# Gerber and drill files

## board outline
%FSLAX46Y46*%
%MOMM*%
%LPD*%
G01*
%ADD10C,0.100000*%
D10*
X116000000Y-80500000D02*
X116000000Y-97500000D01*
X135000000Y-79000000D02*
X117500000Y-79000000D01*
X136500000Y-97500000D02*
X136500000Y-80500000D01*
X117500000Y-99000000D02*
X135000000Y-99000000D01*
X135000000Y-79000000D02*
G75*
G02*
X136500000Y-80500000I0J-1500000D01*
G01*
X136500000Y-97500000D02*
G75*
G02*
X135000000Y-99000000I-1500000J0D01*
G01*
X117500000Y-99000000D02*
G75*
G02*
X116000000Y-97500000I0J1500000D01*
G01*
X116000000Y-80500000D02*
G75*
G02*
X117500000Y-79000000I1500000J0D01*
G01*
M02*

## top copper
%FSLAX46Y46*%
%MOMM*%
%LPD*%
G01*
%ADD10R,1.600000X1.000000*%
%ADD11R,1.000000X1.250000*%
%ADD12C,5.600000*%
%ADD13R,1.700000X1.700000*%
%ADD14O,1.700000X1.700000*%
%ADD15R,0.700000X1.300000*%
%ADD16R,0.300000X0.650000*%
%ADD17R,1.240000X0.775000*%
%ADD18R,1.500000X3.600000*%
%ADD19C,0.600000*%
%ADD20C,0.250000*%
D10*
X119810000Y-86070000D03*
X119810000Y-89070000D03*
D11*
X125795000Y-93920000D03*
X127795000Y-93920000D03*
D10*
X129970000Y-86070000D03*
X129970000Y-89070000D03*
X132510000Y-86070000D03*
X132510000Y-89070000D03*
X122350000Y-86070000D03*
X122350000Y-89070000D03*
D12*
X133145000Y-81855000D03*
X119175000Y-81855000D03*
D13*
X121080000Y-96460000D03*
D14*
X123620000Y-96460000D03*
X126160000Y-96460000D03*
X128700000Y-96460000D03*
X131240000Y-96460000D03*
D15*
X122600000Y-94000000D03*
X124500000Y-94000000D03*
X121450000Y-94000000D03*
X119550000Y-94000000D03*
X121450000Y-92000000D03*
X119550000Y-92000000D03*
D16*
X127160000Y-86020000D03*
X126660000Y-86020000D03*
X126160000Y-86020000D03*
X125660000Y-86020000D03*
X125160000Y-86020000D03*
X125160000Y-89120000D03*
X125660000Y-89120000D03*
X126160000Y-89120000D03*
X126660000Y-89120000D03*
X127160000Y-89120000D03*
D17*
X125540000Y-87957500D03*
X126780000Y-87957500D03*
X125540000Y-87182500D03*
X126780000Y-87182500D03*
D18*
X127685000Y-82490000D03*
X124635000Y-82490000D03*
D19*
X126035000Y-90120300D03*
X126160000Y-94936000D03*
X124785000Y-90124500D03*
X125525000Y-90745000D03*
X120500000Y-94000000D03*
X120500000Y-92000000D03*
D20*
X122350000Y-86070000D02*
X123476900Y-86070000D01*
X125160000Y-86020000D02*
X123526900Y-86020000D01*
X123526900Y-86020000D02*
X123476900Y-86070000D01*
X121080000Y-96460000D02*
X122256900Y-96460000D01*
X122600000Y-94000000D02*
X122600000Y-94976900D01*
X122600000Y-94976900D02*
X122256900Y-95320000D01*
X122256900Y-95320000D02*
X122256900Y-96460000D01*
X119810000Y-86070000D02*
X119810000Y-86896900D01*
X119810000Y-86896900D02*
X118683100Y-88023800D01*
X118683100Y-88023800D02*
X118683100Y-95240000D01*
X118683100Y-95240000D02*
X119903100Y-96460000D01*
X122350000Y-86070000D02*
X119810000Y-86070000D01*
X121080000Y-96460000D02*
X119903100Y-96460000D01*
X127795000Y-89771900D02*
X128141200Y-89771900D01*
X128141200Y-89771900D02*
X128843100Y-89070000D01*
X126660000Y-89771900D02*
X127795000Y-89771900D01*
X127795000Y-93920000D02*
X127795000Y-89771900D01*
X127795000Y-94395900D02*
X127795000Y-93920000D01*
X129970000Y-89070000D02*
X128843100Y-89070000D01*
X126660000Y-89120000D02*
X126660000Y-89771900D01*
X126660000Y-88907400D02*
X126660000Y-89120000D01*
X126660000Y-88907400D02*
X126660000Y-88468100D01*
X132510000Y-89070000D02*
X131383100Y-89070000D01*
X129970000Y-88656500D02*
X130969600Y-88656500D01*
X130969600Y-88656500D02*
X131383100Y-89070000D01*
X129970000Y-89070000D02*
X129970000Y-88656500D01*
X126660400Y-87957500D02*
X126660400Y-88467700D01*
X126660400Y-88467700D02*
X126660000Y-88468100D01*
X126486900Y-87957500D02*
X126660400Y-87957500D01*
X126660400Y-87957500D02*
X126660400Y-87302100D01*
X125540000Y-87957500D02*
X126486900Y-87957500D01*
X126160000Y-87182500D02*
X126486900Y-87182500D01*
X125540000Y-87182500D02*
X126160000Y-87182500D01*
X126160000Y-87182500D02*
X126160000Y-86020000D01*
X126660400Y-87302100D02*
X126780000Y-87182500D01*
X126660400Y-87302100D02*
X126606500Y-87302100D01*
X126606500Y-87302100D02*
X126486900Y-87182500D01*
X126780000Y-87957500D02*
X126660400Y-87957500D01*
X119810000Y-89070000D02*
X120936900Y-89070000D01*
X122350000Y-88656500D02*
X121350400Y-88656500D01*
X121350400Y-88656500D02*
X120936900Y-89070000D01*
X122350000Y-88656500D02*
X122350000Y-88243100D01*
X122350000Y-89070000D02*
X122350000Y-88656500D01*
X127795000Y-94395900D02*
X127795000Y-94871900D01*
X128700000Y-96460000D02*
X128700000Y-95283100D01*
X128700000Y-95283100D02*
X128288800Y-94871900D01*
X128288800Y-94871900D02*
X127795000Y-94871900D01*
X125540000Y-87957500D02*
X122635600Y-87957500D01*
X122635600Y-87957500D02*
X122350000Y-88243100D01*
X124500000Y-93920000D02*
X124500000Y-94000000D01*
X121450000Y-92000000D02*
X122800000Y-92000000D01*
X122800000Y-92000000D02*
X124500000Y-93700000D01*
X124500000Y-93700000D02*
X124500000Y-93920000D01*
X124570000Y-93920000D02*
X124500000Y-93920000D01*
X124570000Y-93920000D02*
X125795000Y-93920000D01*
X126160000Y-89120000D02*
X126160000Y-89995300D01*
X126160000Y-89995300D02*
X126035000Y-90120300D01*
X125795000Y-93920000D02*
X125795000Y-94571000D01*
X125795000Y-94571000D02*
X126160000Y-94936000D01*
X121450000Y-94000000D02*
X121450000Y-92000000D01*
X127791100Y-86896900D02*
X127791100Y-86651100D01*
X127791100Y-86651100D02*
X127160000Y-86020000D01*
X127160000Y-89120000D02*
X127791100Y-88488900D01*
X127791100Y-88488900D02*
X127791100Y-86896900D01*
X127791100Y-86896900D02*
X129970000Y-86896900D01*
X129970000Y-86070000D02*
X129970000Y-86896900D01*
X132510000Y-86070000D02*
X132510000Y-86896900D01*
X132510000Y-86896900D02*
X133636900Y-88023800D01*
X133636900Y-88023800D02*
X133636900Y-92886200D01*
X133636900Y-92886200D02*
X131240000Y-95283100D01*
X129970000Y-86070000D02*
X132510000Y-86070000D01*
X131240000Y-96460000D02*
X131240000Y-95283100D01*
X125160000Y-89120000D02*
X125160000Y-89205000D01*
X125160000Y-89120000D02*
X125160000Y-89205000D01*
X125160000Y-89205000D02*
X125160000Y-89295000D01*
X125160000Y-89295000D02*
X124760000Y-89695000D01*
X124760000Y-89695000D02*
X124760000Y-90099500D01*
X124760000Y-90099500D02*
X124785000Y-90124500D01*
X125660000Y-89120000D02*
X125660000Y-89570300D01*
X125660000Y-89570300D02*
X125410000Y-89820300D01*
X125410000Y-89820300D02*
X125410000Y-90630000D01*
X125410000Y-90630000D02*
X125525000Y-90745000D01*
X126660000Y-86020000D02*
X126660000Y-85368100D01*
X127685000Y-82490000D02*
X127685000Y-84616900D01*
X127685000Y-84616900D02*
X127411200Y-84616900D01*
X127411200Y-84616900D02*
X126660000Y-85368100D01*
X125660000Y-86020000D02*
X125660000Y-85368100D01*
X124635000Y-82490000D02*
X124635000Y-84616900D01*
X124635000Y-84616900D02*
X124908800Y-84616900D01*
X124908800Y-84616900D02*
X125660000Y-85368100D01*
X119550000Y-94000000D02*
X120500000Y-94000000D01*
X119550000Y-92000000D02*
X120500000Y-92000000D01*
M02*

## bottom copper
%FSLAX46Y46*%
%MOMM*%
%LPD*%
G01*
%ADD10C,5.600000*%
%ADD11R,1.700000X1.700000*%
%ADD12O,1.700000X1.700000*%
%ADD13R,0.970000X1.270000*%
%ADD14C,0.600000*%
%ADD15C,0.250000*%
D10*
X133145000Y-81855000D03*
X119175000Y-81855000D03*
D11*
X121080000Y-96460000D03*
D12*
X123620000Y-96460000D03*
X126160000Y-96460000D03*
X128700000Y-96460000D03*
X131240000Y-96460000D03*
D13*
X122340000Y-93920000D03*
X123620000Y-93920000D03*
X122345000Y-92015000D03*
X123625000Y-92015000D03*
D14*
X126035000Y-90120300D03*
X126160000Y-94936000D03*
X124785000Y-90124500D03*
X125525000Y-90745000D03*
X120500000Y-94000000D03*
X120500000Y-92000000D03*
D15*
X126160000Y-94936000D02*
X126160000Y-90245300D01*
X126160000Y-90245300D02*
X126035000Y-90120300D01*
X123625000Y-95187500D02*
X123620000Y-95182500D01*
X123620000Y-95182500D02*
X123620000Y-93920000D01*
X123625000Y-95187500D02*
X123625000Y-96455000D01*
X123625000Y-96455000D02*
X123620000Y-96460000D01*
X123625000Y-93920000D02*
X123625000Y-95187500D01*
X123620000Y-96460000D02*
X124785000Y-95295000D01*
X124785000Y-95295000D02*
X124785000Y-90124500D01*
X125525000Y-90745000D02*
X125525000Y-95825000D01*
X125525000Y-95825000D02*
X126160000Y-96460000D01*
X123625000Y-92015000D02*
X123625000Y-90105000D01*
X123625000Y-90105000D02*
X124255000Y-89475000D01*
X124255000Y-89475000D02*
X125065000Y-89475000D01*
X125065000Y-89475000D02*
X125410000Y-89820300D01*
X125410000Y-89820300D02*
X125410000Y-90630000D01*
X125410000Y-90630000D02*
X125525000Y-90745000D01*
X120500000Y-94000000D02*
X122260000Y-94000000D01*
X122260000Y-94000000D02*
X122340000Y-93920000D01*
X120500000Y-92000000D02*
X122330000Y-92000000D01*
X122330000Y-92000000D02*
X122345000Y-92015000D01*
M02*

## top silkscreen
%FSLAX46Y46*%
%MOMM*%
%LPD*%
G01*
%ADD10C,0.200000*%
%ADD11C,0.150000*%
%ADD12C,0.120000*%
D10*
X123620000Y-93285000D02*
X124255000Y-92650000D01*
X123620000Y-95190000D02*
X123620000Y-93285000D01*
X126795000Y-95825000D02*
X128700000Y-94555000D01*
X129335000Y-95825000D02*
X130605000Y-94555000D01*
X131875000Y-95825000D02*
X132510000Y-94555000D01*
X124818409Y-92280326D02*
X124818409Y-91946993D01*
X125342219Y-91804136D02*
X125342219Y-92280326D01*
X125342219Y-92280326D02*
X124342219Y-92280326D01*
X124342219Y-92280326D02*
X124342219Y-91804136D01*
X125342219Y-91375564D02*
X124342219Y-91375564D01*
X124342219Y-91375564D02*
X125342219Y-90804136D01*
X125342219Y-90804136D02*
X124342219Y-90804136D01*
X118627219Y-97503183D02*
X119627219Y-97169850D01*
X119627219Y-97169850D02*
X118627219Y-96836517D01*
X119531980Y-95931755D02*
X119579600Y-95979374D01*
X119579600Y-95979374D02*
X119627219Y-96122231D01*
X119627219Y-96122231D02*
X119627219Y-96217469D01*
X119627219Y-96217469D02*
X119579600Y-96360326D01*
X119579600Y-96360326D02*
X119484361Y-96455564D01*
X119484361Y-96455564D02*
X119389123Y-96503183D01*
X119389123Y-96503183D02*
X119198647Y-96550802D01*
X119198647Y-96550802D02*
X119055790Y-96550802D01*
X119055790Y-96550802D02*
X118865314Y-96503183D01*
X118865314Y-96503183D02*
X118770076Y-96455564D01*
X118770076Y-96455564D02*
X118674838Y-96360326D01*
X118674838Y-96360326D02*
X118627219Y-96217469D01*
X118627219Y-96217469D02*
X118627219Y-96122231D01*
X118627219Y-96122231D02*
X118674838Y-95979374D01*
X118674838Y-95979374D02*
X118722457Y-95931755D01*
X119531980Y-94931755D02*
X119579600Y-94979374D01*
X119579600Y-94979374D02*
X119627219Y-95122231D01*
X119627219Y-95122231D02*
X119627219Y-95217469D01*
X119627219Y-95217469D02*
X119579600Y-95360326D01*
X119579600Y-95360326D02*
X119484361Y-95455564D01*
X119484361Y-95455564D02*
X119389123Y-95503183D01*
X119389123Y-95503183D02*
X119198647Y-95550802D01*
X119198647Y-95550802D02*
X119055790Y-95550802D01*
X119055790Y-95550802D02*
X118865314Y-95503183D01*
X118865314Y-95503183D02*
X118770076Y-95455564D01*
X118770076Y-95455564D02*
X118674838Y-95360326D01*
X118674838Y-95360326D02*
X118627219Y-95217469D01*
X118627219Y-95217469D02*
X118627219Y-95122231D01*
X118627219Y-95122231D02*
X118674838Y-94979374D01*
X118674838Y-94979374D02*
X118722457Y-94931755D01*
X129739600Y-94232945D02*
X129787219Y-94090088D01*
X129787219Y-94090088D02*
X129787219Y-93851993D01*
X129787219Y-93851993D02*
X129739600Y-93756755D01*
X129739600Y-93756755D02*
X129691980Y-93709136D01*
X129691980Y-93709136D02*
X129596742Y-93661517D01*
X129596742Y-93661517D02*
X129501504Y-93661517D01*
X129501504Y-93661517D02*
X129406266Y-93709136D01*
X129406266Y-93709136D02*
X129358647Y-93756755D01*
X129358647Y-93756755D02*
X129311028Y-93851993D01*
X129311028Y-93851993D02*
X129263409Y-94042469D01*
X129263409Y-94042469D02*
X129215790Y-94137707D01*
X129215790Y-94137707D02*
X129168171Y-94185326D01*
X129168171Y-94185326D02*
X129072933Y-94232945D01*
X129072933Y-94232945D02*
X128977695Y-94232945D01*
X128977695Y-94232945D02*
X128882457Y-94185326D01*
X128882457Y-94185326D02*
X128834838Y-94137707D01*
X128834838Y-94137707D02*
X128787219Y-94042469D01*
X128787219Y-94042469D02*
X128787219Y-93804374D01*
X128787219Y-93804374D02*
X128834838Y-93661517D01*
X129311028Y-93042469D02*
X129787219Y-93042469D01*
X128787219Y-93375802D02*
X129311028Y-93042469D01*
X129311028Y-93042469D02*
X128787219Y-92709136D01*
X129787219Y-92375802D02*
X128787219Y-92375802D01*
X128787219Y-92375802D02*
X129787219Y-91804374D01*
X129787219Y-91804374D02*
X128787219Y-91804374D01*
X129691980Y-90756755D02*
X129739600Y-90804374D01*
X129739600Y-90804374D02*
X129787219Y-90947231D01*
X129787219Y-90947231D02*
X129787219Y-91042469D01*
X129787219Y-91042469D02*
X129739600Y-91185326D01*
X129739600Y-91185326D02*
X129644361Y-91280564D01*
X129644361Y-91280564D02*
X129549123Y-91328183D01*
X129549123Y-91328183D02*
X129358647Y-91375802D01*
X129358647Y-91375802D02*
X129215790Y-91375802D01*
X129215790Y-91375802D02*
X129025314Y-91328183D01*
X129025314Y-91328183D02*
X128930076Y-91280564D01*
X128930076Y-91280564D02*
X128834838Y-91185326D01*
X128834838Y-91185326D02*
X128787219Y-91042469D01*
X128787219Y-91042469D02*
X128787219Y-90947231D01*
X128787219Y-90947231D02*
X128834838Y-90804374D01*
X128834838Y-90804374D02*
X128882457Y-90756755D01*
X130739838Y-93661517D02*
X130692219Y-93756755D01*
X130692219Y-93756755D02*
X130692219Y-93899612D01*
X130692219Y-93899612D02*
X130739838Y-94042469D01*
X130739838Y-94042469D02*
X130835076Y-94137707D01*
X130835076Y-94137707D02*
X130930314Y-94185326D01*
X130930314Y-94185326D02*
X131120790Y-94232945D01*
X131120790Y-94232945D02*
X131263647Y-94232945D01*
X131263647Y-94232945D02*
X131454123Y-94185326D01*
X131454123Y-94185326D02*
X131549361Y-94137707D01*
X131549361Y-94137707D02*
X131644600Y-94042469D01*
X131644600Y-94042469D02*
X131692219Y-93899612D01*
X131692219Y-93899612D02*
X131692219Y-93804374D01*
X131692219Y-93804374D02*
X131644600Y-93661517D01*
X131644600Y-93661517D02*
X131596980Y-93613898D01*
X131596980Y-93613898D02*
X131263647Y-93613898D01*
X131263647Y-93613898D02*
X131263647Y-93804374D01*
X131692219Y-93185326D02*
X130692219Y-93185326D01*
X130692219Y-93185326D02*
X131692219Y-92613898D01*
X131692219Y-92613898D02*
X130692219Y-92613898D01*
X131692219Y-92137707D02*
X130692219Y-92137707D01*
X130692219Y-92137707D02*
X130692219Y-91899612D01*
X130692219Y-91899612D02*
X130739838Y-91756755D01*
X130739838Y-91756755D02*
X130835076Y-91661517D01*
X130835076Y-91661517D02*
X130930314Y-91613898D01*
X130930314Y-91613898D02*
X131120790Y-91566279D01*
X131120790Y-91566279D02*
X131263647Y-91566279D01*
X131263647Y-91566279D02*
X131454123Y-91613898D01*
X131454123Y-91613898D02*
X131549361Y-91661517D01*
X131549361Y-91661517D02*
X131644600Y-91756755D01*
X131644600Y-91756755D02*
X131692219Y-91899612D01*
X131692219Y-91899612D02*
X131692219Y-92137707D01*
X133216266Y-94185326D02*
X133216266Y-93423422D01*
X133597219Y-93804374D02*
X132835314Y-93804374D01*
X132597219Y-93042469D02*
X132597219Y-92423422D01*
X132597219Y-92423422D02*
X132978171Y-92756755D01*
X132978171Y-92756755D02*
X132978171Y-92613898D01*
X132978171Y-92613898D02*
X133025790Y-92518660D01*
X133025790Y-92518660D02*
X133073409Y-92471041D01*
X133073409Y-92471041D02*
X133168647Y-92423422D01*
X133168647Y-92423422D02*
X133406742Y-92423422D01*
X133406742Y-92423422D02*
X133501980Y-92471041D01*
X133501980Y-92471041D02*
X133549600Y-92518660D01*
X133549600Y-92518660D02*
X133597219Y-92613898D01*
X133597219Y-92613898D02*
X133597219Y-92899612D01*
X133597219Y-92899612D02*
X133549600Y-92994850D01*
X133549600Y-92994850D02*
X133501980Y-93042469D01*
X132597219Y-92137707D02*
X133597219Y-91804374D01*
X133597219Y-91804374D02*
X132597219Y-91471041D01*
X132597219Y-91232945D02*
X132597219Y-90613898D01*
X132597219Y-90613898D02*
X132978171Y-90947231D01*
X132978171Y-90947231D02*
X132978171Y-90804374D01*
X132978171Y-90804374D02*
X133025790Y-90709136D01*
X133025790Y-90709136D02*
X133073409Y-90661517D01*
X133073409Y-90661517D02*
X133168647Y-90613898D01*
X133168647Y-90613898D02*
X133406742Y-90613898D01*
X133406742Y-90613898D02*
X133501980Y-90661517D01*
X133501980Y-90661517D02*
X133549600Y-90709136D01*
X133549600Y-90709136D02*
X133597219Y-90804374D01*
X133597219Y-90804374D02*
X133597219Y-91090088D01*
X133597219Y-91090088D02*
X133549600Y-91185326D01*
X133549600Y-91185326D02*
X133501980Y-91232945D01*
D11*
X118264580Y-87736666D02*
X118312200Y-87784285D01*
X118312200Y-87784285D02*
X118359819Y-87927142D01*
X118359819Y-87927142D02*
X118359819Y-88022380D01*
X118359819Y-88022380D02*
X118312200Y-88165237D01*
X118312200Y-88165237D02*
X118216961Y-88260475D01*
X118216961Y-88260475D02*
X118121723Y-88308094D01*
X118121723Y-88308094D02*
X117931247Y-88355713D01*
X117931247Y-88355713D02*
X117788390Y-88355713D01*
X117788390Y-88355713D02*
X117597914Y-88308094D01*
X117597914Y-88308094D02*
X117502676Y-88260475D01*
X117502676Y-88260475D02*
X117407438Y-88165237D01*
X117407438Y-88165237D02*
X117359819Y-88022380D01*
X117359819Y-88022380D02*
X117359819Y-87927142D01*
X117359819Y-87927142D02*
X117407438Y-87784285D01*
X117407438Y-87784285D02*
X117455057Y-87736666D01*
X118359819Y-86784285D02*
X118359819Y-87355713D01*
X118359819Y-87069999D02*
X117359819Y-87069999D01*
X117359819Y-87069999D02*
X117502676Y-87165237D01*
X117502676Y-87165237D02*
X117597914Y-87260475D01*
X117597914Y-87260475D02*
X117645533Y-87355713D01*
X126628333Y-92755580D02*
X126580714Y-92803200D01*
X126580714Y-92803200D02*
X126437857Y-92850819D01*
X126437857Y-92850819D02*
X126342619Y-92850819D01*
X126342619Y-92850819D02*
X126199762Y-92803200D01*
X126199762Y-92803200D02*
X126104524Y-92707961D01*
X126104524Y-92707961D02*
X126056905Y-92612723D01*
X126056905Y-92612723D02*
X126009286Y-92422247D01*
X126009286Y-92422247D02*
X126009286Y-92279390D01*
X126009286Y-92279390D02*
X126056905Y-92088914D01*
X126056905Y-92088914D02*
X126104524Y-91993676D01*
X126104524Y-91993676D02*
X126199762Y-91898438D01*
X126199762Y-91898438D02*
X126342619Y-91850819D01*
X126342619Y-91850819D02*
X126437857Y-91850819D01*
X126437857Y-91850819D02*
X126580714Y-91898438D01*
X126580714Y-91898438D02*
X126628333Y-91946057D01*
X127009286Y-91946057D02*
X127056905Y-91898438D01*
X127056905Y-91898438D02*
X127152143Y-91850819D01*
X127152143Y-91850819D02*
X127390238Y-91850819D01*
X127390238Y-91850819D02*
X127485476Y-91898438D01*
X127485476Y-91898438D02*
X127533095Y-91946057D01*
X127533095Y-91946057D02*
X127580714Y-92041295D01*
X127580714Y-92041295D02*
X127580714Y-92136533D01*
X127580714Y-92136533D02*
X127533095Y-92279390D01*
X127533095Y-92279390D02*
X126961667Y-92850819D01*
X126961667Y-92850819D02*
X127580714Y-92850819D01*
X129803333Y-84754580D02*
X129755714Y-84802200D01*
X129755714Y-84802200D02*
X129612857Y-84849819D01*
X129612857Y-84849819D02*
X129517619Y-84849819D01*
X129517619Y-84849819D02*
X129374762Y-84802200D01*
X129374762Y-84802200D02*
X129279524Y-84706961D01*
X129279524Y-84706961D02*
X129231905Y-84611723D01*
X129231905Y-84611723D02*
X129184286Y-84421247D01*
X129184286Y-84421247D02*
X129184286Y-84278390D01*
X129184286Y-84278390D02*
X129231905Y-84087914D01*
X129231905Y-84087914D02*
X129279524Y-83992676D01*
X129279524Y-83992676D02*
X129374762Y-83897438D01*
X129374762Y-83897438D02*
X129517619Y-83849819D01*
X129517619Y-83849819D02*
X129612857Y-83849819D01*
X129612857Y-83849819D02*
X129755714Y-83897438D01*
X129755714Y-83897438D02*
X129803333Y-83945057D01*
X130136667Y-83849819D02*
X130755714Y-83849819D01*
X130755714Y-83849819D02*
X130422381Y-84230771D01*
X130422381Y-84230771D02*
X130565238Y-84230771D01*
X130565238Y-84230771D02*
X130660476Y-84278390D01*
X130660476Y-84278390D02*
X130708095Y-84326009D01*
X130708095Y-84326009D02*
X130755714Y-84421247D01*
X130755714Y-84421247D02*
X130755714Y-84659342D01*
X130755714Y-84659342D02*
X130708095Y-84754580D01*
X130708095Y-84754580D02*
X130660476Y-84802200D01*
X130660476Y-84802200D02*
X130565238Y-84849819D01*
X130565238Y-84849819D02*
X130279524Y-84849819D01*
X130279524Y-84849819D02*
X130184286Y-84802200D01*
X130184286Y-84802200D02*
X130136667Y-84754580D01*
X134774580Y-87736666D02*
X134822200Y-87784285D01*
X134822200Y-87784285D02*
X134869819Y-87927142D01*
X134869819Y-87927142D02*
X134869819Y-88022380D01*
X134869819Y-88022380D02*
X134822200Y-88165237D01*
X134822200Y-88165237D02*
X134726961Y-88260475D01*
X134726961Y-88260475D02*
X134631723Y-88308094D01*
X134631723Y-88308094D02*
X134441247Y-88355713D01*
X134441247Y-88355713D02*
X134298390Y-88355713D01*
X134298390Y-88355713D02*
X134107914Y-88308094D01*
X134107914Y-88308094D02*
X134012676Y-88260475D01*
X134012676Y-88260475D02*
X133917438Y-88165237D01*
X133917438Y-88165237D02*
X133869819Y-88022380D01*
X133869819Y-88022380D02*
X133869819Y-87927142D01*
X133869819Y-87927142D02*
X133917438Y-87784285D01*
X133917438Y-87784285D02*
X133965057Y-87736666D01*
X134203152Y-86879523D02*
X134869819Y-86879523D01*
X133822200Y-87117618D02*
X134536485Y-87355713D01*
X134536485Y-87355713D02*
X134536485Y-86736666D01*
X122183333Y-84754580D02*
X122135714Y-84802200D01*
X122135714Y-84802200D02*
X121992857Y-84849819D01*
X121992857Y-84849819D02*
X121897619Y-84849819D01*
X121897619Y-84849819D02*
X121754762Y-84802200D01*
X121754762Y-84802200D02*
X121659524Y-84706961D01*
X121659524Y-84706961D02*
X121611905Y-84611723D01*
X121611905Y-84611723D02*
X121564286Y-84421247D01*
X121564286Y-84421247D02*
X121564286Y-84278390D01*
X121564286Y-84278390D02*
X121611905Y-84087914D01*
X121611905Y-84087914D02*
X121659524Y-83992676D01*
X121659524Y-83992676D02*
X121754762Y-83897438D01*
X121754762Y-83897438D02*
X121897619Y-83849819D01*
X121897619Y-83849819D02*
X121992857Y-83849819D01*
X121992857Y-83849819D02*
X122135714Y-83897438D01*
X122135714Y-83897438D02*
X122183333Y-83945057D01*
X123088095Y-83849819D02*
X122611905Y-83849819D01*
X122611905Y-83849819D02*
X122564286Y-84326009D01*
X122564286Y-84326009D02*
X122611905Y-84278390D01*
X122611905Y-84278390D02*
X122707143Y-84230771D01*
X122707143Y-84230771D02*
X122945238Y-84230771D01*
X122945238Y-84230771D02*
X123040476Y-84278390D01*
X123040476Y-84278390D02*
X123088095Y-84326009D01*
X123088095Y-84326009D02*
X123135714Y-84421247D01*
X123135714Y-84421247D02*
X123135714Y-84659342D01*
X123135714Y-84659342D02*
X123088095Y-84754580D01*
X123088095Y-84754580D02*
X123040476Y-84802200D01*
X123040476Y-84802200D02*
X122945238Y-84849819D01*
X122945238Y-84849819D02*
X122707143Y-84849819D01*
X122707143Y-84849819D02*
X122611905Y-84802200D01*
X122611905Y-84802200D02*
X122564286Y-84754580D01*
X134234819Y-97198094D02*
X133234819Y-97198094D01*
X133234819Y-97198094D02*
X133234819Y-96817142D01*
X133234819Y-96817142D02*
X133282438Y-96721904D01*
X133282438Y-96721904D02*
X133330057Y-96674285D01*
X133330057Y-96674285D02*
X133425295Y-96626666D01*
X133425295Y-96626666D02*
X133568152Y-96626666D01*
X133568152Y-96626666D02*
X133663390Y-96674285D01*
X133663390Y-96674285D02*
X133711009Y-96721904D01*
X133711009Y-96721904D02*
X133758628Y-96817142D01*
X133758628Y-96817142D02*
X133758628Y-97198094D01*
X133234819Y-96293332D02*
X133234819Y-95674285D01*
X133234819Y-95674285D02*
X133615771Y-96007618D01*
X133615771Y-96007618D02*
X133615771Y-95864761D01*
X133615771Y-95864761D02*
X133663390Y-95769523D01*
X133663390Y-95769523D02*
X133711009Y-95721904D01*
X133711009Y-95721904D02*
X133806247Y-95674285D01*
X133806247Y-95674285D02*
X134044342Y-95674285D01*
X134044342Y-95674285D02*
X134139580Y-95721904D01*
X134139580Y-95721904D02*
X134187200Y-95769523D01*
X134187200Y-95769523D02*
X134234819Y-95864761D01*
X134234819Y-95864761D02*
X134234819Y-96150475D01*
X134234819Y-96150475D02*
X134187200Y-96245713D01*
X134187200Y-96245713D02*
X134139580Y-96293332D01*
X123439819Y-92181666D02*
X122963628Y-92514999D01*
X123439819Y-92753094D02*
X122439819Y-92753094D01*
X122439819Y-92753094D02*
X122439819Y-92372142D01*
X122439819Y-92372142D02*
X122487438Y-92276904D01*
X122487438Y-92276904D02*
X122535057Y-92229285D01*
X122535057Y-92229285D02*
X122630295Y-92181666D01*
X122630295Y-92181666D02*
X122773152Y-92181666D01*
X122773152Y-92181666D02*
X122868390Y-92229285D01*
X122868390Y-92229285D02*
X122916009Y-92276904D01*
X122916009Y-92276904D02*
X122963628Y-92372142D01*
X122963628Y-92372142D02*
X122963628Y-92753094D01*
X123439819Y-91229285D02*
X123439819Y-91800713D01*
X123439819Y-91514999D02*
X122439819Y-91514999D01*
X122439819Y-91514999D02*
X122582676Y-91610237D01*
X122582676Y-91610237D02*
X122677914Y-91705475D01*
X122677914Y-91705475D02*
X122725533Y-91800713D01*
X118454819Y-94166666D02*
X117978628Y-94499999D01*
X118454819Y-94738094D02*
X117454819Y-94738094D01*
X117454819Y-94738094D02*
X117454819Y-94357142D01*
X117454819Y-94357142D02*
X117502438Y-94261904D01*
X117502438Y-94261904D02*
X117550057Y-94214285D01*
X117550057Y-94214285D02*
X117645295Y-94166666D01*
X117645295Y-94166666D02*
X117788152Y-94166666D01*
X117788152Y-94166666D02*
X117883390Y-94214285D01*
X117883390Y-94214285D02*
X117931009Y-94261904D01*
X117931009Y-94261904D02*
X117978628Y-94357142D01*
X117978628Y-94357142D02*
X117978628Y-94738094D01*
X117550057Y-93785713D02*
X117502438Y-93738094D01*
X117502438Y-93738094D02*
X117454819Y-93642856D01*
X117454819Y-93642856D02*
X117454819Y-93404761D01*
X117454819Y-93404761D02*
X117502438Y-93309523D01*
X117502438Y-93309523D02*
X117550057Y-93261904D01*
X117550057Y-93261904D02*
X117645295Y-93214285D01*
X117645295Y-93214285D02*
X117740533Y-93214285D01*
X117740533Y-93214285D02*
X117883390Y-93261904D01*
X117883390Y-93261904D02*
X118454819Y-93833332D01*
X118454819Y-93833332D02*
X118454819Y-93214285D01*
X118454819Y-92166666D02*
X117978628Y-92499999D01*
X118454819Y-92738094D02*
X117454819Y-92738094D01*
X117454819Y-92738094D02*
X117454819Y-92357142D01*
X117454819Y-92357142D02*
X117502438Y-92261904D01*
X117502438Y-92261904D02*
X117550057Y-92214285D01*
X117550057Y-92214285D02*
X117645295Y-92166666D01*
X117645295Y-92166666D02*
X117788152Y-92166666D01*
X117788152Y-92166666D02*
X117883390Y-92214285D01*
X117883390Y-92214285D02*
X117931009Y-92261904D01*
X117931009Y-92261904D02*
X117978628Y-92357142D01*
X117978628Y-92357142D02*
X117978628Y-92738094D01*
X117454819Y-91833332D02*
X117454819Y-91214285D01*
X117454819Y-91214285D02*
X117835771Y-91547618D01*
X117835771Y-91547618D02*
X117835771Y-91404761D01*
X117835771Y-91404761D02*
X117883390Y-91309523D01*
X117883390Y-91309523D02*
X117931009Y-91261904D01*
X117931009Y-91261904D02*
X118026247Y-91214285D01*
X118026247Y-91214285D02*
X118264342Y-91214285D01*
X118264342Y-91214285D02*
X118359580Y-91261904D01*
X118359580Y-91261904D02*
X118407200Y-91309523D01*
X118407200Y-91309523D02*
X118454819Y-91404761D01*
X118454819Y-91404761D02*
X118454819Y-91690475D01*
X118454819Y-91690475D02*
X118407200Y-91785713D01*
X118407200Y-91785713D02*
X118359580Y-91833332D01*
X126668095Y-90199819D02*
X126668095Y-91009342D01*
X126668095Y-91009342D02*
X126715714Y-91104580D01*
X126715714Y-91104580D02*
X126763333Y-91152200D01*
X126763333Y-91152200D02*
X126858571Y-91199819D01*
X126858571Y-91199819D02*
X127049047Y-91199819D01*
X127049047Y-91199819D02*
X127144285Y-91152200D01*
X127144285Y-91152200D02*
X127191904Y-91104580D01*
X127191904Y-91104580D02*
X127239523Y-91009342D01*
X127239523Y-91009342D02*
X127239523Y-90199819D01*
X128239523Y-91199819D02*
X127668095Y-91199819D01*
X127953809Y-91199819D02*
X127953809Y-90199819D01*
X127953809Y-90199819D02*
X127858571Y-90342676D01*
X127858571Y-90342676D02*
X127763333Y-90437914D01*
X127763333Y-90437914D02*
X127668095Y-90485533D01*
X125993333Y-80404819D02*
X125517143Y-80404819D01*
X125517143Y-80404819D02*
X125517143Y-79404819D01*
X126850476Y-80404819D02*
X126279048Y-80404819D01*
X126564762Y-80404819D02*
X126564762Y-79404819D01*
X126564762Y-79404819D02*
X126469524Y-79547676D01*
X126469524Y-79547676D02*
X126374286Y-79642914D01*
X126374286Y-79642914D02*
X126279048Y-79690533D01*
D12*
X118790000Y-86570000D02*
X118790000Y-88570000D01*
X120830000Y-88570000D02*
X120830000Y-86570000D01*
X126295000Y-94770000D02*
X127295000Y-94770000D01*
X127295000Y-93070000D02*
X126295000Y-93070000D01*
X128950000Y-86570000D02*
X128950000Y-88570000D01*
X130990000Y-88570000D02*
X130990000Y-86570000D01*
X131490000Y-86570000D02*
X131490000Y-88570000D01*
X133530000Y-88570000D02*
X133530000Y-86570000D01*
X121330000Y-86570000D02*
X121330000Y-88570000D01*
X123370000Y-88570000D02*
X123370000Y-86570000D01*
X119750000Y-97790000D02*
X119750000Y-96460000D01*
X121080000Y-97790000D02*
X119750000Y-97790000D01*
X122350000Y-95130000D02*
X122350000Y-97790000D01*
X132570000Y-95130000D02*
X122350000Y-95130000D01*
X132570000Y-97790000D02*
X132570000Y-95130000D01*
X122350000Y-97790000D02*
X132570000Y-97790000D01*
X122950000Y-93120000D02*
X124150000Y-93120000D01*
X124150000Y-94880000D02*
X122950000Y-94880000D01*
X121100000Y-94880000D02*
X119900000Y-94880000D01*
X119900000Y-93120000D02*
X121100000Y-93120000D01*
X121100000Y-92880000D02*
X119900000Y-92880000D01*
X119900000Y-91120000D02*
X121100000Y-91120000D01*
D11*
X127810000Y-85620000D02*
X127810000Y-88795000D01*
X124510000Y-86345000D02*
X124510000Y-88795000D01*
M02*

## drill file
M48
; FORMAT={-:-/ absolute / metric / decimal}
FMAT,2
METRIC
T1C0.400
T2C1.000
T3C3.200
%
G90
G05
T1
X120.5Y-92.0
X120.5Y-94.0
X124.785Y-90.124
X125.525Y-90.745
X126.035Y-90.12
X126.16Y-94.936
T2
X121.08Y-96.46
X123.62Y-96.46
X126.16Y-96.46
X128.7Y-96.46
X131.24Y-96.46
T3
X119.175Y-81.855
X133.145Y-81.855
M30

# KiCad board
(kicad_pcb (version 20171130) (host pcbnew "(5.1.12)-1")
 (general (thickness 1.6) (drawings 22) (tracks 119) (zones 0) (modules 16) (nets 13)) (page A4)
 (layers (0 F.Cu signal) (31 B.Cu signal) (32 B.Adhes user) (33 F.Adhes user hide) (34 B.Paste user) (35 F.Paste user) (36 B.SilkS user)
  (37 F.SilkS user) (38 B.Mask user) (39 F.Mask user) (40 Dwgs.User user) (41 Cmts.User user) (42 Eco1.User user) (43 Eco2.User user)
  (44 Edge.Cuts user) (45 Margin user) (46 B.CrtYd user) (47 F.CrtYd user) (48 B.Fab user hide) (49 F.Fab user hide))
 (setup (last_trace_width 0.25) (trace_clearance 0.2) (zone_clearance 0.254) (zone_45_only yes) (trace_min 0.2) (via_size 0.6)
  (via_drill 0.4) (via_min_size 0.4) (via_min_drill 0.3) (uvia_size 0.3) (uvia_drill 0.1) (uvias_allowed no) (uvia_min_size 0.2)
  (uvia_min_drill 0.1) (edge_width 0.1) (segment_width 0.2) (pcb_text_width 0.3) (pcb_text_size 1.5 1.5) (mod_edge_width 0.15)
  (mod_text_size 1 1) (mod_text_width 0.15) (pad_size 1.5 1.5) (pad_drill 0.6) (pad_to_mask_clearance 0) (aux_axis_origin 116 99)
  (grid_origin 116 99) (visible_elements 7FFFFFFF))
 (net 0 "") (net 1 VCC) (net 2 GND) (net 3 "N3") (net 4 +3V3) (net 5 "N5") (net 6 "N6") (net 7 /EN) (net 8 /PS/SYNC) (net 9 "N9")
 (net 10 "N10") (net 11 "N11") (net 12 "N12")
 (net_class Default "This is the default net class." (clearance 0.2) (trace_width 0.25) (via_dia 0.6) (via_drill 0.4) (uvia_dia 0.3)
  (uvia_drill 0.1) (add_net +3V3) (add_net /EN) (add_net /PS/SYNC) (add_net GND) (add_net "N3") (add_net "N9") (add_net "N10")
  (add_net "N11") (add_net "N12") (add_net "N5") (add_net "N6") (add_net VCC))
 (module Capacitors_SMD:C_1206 (layer F.Cu) (at 119.81 87.57 270)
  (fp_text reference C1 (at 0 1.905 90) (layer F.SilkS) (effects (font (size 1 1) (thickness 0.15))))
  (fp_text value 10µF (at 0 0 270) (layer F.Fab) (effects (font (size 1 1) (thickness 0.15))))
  (fp_line (start -1 1.02) (end 1 1.02) (layer F.SilkS) (width 0.12))
  (fp_line (start 1 -1.02) (end -1 -1.02) (layer F.SilkS) (width 0.12))
  (pad 1 smd rect (at -1.5 0 270) (size 1 1.6) (layers F.Cu F.Paste F.Mask) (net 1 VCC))
  (pad 2 smd rect (at 1.5 0 270) (size 1 1.6) (layers F.Cu F.Paste F.Mask) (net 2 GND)))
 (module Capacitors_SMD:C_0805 (layer F.Cu) (at 126.795 93.92)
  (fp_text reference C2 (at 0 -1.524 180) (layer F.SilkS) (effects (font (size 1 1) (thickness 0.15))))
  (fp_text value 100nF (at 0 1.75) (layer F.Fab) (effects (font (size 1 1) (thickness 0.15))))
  (fp_line (start -0.5 0.85) (end 0.5 0.85) (layer F.SilkS) (width 0.12))
  (fp_line (start 0.5 -0.85) (end -0.5 -0.85) (layer F.SilkS) (width 0.12))
  (pad 1 smd rect (at -1 0) (size 1 1.25) (layers F.Cu F.Paste F.Mask) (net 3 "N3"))
  (pad 2 smd rect (at 1 0) (size 1 1.25) (layers F.Cu F.Paste F.Mask) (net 2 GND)))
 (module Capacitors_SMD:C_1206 (layer F.Cu) (at 129.97 87.57 270)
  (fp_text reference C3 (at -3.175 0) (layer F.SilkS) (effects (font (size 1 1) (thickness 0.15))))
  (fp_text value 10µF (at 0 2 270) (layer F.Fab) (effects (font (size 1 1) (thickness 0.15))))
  (fp_line (start -1 1.02) (end 1 1.02) (layer F.SilkS) (width 0.12))
  (fp_line (start 1 -1.02) (end -1 -1.02) (layer F.SilkS) (width 0.12))
  (pad 1 smd rect (at -1.5 0 270) (size 1 1.6) (layers F.Cu F.Paste F.Mask) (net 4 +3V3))
  (pad 2 smd rect (at 1.5 0 270) (size 1 1.6) (layers F.Cu F.Paste F.Mask) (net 2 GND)))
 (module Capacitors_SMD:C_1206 (layer F.Cu) (at 132.51 87.57 270)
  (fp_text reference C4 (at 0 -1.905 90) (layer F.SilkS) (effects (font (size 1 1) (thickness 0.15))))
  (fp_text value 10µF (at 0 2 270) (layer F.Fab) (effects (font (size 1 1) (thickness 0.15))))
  (fp_line (start -1 1.02) (end 1 1.02) (layer F.SilkS) (width 0.12))
  (fp_line (start 1 -1.02) (end -1 -1.02) (layer F.SilkS) (width 0.12))
  (pad 1 smd rect (at -1.5 0 270) (size 1 1.6) (layers F.Cu F.Paste F.Mask) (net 4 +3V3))
  (pad 2 smd rect (at 1.5 0 270) (size 1 1.6) (layers F.Cu F.Paste F.Mask) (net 2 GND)))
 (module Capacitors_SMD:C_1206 (layer F.Cu) (at 122.35 87.57 270)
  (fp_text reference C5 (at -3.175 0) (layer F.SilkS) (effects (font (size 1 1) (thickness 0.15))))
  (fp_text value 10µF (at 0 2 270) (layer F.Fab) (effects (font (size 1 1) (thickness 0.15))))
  (fp_line (start -1 1.02) (end 1 1.02) (layer F.SilkS) (width 0.12))
  (fp_line (start 1 -1.02) (end -1 -1.02) (layer F.SilkS) (width 0.12))
  (pad 1 smd rect (at -1.5 0 270) (size 1 1.6) (layers F.Cu F.Paste F.Mask) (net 1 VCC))
  (pad 2 smd rect (at 1.5 0 270) (size 1 1.6) (layers F.Cu F.Paste F.Mask) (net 2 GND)))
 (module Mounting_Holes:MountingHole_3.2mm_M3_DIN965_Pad (layer F.Cu) (at 133.145 81.855)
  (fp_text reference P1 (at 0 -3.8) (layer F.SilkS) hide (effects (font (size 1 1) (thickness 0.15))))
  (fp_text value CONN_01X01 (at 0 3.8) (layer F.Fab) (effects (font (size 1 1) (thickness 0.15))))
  (pad 1 thru_hole circle (at 0 0) (size 5.6 5.6) (drill 3.2) (layers *.Cu *.Mask) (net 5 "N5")))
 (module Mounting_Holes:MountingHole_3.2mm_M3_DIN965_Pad (layer F.Cu) (at 119.175 81.855)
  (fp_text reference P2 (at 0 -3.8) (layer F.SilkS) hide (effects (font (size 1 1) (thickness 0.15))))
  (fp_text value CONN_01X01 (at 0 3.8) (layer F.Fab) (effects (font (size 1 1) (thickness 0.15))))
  (pad 1 thru_hole circle (at 0 0) (size 5.6 5.6) (drill 3.2) (layers *.Cu *.Mask) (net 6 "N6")))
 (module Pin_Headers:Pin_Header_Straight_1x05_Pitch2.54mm (layer F.Cu) (at 121.08 96.46 90)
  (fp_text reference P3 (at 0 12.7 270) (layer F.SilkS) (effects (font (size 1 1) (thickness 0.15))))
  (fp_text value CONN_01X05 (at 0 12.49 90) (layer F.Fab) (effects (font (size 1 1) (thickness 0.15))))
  (fp_line (start -1.33 -1.33) (end 0 -1.33) (layer F.SilkS) (width 0.12))
  (fp_line (start -1.33 0) (end -1.33 -1.33) (layer F.SilkS) (width 0.12))
  (fp_line (start 1.33 1.27) (end -1.33 1.27) (layer F.SilkS) (width 0.12))
  (fp_line (start 1.33 11.49) (end 1.33 1.27) (layer F.SilkS) (width 0.12))
  (fp_line (start -1.33 11.49) (end 1.33 11.49) (layer F.SilkS) (width 0.12))
  (fp_line (start -1.33 1.27) (end -1.33 11.49) (layer F.SilkS) (width 0.12))
  (pad 1 thru_hole rect (at 0 0 90) (size 1.7 1.7) (drill 1) (layers *.Cu *.Mask) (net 1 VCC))
  (pad 2 thru_hole oval (at 0 2.54 90) (size 1.7 1.7) (drill 1) (layers *.Cu *.Mask) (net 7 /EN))
  (pad 3 thru_hole oval (at 0 5.08 90) (size 1.7 1.7) (drill 1) (layers *.Cu *.Mask) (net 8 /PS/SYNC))
  (pad 4 thru_hole oval (at 0 7.62 90) (size 1.7 1.7) (drill 1) (layers *.Cu *.Mask) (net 2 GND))
  (pad 5 thru_hole oval (at 0 10.16 90) (size 1.7 1.7) (drill 1) (layers *.Cu *.Mask) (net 4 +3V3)))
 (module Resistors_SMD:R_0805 (layer F.Cu) (at 123.55 94)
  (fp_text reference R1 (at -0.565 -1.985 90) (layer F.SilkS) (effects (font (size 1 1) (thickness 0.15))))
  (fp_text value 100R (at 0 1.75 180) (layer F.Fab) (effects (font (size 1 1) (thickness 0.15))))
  (fp_line (start -0.6 -0.88) (end 0.6 -0.88) (layer F.SilkS) (width 0.12))
  (fp_line (start 0.6 0.88) (end -0.6 0.88) (layer F.SilkS) (width 0.12))
  (pad 1 smd rect (at -0.95 0) (size 0.7 1.3) (layers F.Cu F.Paste F.Mask) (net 1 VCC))
  (pad 2 smd rect (at 0.95 0) (size 0.7 1.3) (layers F.Cu F.Paste F.Mask) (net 3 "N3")))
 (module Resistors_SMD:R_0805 (layer F.Cu) (at 120.5 94 180)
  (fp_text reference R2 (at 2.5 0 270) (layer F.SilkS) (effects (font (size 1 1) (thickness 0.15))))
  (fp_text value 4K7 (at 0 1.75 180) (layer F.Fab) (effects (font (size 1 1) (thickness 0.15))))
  (fp_line (start -0.6 -0.88) (end 0.6 -0.88) (layer F.SilkS) (width 0.12))
  (fp_line (start 0.6 0.88) (end -0.6 0.88) (layer F.SilkS) (width 0.12))
  (pad 1 smd rect (at -0.95 0 180) (size 0.7 1.3) (layers F.Cu F.Paste F.Mask) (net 3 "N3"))
  (pad 2 smd rect (at 0.95 0 180) (size 0.7 1.3) (layers F.Cu F.Paste F.Mask) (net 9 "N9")))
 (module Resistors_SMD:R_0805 (layer F.Cu) (at 120.5 92 180)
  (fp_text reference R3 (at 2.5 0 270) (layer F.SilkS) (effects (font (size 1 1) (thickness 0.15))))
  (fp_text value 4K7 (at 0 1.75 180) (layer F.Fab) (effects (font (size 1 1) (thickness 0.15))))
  (fp_line (start -0.6 -0.88) (end 0.6 -0.88) (layer F.SilkS) (width 0.12))
  (fp_line (start 0.6 0.88) (end -0.6 0.88) (layer F.SilkS) (width 0.12))
  (pad 1 smd rect (at -0.95 0 180) (size 0.7 1.3) (layers F.Cu F.Paste F.Mask) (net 3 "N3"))
  (pad 2 smd rect (at 0.95 0 180) (size 0.7 1.3) (layers F.Cu F.Paste F.Mask) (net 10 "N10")))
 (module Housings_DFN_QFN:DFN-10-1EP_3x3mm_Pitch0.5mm (layer F.Cu) (at 126.16 87.57 270)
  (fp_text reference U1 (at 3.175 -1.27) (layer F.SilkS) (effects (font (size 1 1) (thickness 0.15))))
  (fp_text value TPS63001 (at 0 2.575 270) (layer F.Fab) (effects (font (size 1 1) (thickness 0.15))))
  (fp_line (start -1.95 -1.65) (end 1.225 -1.65) (layer F.SilkS) (width 0.15))
  (fp_line (start -1.225 1.65) (end 1.225 1.65) (layer F.SilkS) (width 0.15))
  (pad 1 smd rect (at -1.55 -1 270) (size 0.65 0.3) (layers F.Cu F.Paste F.Mask) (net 4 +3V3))
  (pad 2 smd rect (at -1.55 -0.5 270) (size 0.65 0.3) (layers F.Cu F.Paste F.Mask) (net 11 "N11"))
  (pad 3 smd rect (at -1.55 0 270) (size 0.65 0.3) (layers F.Cu F.Paste F.Mask) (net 2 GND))
  (pad 4 smd rect (at -1.55 0.5 270) (size 0.65 0.3) (layers F.Cu F.Paste F.Mask) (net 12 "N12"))
  (pad 5 smd rect (at -1.55 1 270) (size 0.65 0.3) (layers F.Cu F.Paste F.Mask) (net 1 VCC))
  (pad 6 smd rect (at 1.55 1 270) (size 0.65 0.3) (layers F.Cu F.Paste F.Mask) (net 7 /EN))
  (pad 7 smd rect (at 1.55 0.5 270) (size 0.65 0.3) (layers F.Cu F.Paste F.Mask) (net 8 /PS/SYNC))
  (pad 8 smd rect (at 1.55 0 270) (size 0.65 0.3) (layers F.Cu F.Paste F.Mask) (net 3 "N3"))
  (pad 9 smd rect (at 1.55 -0.5 270) (size 0.65 0.3) (layers F.Cu F.Paste F.Mask) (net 2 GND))
  (pad 10 smd rect (at 1.55 -1 270) (size 0.65 0.3) (layers F.Cu F.Paste F.Mask) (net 4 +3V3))
  (pad 11 smd rect (at 0.3875 0.62 270) (size 0.775 1.24) (layers F.Cu F.Paste F.Mask) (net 2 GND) (solder_paste_margin_ratio -0.2))
  (pad 11 smd rect (at 0.3875 -0.62 270) (size 0.775 1.24) (layers F.Cu F.Paste F.Mask) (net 2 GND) (solder_paste_margin_ratio -0.2))
  (pad 11 smd rect (at -0.3875 0.62 270) (size 0.775 1.24) (layers F.Cu F.Paste F.Mask) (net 2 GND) (solder_paste_margin_ratio -0.2))
  (pad 11 smd rect (at -0.3875 -0.62 270) (size 0.775 1.24) (layers F.Cu F.Paste F.Mask) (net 2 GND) (solder_paste_margin_ratio -0.2)))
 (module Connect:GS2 (layer B.Cu) (at 122.98 93.92 270)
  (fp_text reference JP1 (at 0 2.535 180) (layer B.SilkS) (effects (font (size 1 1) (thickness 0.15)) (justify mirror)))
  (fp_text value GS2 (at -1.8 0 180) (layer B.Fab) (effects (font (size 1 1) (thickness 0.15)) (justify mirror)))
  (pad 1 smd rect (at 0 0.64 270) (size 1.27 0.97) (layers B.Cu B.Paste B.Mask) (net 9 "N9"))
  (pad 2 smd rect (at 0 -0.64 270) (size 1.27 0.97) (layers B.Cu B.Paste B.Mask) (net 7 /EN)))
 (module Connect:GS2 (layer B.Cu) (at 122.985 92.015 270)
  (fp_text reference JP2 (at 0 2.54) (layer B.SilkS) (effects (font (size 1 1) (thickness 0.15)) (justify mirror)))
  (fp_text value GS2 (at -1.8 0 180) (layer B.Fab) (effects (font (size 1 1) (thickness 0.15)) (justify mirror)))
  (pad 1 smd rect (at 0 0.64 270) (size 1.27 0.97) (layers B.Cu B.Paste B.Mask) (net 10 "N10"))
  (pad 2 smd rect (at 0 -0.64 270) (size 1.27 0.97) (layers B.Cu B.Paste B.Mask) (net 8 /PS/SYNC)))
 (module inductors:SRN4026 (layer F.Cu) (at 126.16 82.49 180)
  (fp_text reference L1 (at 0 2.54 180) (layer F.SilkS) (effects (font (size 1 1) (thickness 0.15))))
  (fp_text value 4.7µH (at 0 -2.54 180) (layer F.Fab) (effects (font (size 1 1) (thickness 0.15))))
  (pad 1 smd rect (at -1.525 0 270) (size 3.6 1.5) (layers F.Cu F.Paste F.Mask) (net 11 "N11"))
  (pad 2 smd rect (at 1.525 0 270) (size 3.6 1.5) (layers F.Cu F.Paste F.Mask) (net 12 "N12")))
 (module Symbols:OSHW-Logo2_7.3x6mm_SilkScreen (layer B.Cu) (at 119.5 89 90)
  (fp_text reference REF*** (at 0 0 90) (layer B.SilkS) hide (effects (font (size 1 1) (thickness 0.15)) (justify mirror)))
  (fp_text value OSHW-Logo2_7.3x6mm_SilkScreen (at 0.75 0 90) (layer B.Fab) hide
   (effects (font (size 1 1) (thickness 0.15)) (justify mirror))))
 (gr_line (start 123.62 93.285) (end 124.255 92.65) (layer F.SilkS) (width 0.2))
 (gr_line (start 123.62 95.19) (end 123.62 93.285) (layer F.SilkS) (width 0.2))
 (gr_line (start 126.795 95.825) (end 128.7 94.555) (layer F.SilkS) (width 0.2))
 (gr_line (start 129.335 95.825) (end 130.605 94.555) (layer F.SilkS) (width 0.2))
 (gr_line (start 131.875 95.825) (end 132.51 94.555) (layer F.SilkS) (width 0.2))
 (gr_line (start 116 80.5) (end 116 97.5) (angle 90) (layer Edge.Cuts) (width 0.1))
 (gr_line (start 135 79) (end 117.5 79) (angle 90) (layer Edge.Cuts) (width 0.1))
 (gr_line (start 136.5 97.5) (end 136.5 80.5) (angle 90) (layer Edge.Cuts) (width 0.1))
 (gr_line (start 117.5 99) (end 135 99) (angle 90) (layer Edge.Cuts) (width 0.1))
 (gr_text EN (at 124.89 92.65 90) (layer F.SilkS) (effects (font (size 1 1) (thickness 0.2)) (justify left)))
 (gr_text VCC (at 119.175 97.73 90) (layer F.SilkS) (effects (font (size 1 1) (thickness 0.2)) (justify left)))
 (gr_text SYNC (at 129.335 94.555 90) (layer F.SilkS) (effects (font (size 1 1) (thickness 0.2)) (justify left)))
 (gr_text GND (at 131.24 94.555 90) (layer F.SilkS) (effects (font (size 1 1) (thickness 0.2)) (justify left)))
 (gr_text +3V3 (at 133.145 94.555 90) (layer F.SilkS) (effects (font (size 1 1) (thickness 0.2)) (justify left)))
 (gr_arc (start 135 80.5) (end 135 79) (angle 90) (layer Edge.Cuts) (width 0.1))
 (gr_arc (start 135 97.5) (end 136.5 97.5) (angle 90) (layer Edge.Cuts) (width 0.1))
 (gr_arc (start 117.5 97.5) (end 117.5 99) (angle 90) (layer Edge.Cuts) (width 0.1))
 (gr_arc (start 117.5 80.5) (end 116 80.5) (angle 90) (layer Edge.Cuts) (width 0.1))
 (segment (start 122.35 86.07) (end 123.4769 86.07) (width 0.25) (layer F.Cu) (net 1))
 (segment (start 125.16 86.02) (end 123.5269 86.02) (width 0.25) (layer F.Cu) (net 1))
 (segment (start 123.5269 86.02) (end 123.4769 86.07) (width 0.25) (layer F.Cu) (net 1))
 (segment (start 121.08 96.46) (end 122.2569 96.46) (width 0.25) (layer F.Cu) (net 1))
 (segment (start 122.6 94) (end 122.6 94.9769) (width 0.25) (layer F.Cu) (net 1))
 (segment (start 122.6 94.9769) (end 122.2569 95.32) (width 0.25) (layer F.Cu) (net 1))
 (segment (start 122.2569 95.32) (end 122.2569 96.46) (width 0.25) (layer F.Cu) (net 1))
 (segment (start 119.81 86.07) (end 119.81 86.8969) (width 0.25) (layer F.Cu) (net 1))
 (segment (start 119.81 86.8969) (end 118.6831 88.0238) (width 0.25) (layer F.Cu) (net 1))
 (segment (start 118.6831 88.0238) (end 118.6831 95.24) (width 0.25) (layer F.Cu) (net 1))
 (segment (start 118.6831 95.24) (end 119.9031 96.46) (width 0.25) (layer F.Cu) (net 1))
 (segment (start 122.35 86.07) (end 119.81 86.07) (width 0.25) (layer F.Cu) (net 1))
 (segment (start 121.08 96.46) (end 119.9031 96.46) (width 0.25) (layer F.Cu) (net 1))
 (segment (start 127.795 89.7719) (end 128.1412 89.7719) (width 0.25) (layer F.Cu) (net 2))
 (segment (start 128.1412 89.7719) (end 128.8431 89.07) (width 0.25) (layer F.Cu) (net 2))
 (segment (start 126.66 89.7719) (end 127.795 89.7719) (width 0.25) (layer F.Cu) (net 2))
 (segment (start 127.795 93.92) (end 127.795 89.7719) (width 0.25) (layer F.Cu) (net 2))
 (segment (start 127.795 94.3959) (end 127.795 93.92) (width 0.25) (layer F.Cu) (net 2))
 (segment (start 129.97 89.07) (end 128.8431 89.07) (width 0.25) (layer F.Cu) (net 2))
 (segment (start 126.66 89.12) (end 126.66 89.7719) (width 0.25) (layer F.Cu) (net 2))
 (segment (start 126.66 88.9074) (end 126.66 89.12) (width 0.25) (layer F.Cu) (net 2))
 (segment (start 126.66 88.9074) (end 126.66 88.4681) (width 0.25) (layer F.Cu) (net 2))
 (segment (start 132.51 89.07) (end 131.3831 89.07) (width 0.25) (layer F.Cu) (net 2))
 (segment (start 129.97 88.6565) (end 130.9696 88.6565) (width 0.25) (layer F.Cu) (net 2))
 (segment (start 130.9696 88.6565) (end 131.3831 89.07) (width 0.25) (layer F.Cu) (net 2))
 (segment (start 129.97 89.07) (end 129.97 88.6565) (width 0.25) (layer F.Cu) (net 2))
 (segment (start 126.6604 87.9575) (end 126.6604 88.4677) (width 0.25) (layer F.Cu) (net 2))
 (segment (start 126.6604 88.4677) (end 126.66 88.4681) (width 0.25) (layer F.Cu) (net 2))
 (segment (start 126.4869 87.9575) (end 126.6604 87.9575) (width 0.25) (layer F.Cu) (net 2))
 (segment (start 126.6604 87.9575) (end 126.6604 87.3021) (width 0.25) (layer F.Cu) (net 2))
 (segment (start 125.54 87.9575) (end 126.4869 87.9575) (width 0.25) (layer F.Cu) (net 2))
 (segment (start 126.16 87.1825) (end 126.4869 87.1825) (width 0.25) (layer F.Cu) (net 2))
 (segment (start 125.54 87.1825) (end 126.16 87.1825) (width 0.25) (layer F.Cu) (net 2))
 (segment (start 126.16 87.1825) (end 126.16 86.02) (width 0.25) (layer F.Cu) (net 2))
 (segment (start 126.6604 87.3021) (end 126.78 87.1825) (width 0.25) (layer F.Cu) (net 2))
 (segment (start 126.6604 87.3021) (end 126.6065 87.3021) (width 0.25) (layer F.Cu) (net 2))
 (segment (start 126.6065 87.3021) (end 126.4869 87.1825) (width 0.25) (layer F.Cu) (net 2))
 (segment (start 126.78 87.9575) (end 126.6604 87.9575) (width 0.25) (layer F.Cu) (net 2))
 (segment (start 119.81 89.07) (end 120.9369 89.07) (width 0.25) (layer F.Cu) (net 2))
 (segment (start 122.35 88.6565) (end 121.3504 88.6565) (width 0.25) (layer F.Cu) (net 2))
 (segment (start 121.3504 88.6565) (end 120.9369 89.07) (width 0.25) (layer F.Cu) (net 2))
 (segment (start 122.35 88.6565) (end 122.35 88.2431) (width 0.25) (layer F.Cu) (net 2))
 (segment (start 122.35 89.07) (end 122.35 88.6565) (width 0.25) (layer F.Cu) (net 2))
 (segment (start 127.795 94.3959) (end 127.795 94.8719) (width 0.25) (layer F.Cu) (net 2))
 (segment (start 128.7 96.46) (end 128.7 95.2831) (width 0.25) (layer F.Cu) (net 2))
 (segment (start 128.7 95.2831) (end 128.2888 94.8719) (width 0.25) (layer F.Cu) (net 2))
 (segment (start 128.2888 94.8719) (end 127.795 94.8719) (width 0.25) (layer F.Cu) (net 2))
 (segment (start 125.54 87.9575) (end 122.6356 87.9575) (width 0.25) (layer F.Cu) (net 2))
 (segment (start 122.6356 87.9575) (end 122.35 88.2431) (width 0.25) (layer F.Cu) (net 2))
 (segment (start 124.5 93.92) (end 124.5 94) (width 0.25) (layer F.Cu) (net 3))
 (segment (start 121.45 92) (end 122.8 92) (width 0.25) (layer F.Cu) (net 3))
 (segment (start 122.8 92) (end 124.5 93.7) (width 0.25) (layer F.Cu) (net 3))
 (segment (start 124.5 93.7) (end 124.5 93.92) (width 0.25) (layer F.Cu) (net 3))
 (segment (start 124.57 93.92) (end 124.5 93.92) (width 0.25) (layer F.Cu) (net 3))
 (segment (start 124.57 93.92) (end 125.795 93.92) (width 0.25) (layer F.Cu) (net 3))
 (segment (start 126.16 89.12) (end 126.16 89.9953) (width 0.25) (layer F.Cu) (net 3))
 (segment (start 126.16 89.9953) (end 126.035 90.1203) (width 0.25) (layer F.Cu) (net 3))
 (segment (start 125.795 93.92) (end 125.795 94.571) (width 0.25) (layer F.Cu) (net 3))
 (segment (start 125.795 94.571) (end 126.16 94.936) (width 0.25) (layer F.Cu) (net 3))
 (segment (start 126.16 94.936) (end 126.16 90.2453) (width 0.25) (layer B.Cu) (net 3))
 (segment (start 126.16 90.2453) (end 126.035 90.1203) (width 0.25) (layer B.Cu) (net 3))
 (segment (start 121.45 94) (end 121.45 92) (width 0.25) (layer F.Cu) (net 3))
 (via (at 126.035 90.1203) (size 0.6) (layers F.Cu B.Cu) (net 3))
 (via (at 126.16 94.936) (size 0.6) (layers F.Cu B.Cu) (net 3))
 (segment (start 127.7911 86.8969) (end 127.7911 86.6511) (width 0.25) (layer F.Cu) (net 4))
 (segment (start 127.7911 86.6511) (end 127.16 86.02) (width 0.25) (layer F.Cu) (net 4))
 (segment (start 127.16 89.12) (end 127.7911 88.4889) (width 0.25) (layer F.Cu) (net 4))
 (segment (start 127.7911 88.4889) (end 127.7911 86.8969) (width 0.25) (layer F.Cu) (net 4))
 (segment (start 127.7911 86.8969) (end 129.97 86.8969) (width 0.25) (layer F.Cu) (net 4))
 (segment (start 129.97 86.07) (end 129.97 86.8969) (width 0.25) (layer F.Cu) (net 4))
 (segment (start 132.51 86.07) (end 132.51 86.8969) (width 0.25) (layer F.Cu) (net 4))
 (segment (start 132.51 86.8969) (end 133.6369 88.0238) (width 0.25) (layer F.Cu) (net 4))
 (segment (start 133.6369 88.0238) (end 133.6369 92.8862) (width 0.25) (layer F.Cu) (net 4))
 (segment (start 133.6369 92.8862) (end 131.24 95.2831) (width 0.25) (layer F.Cu) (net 4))
 (segment (start 129.97 86.07) (end 132.51 86.07) (width 0.25) (layer F.Cu) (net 4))
 (segment (start 131.24 96.46) (end 131.24 95.2831) (width 0.25) (layer F.Cu) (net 4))
 (segment (start 123.625 95.1875) (end 123.62 95.1825) (width 0.25) (layer B.Cu) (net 7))
 (segment (start 123.62 95.1825) (end 123.62 93.92) (width 0.25) (layer B.Cu) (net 7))
 (segment (start 123.625 95.1875) (end 123.625 96.455) (width 0.25) (layer B.Cu) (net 7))
 (segment (start 123.625 96.455) (end 123.62 96.46) (width 0.25) (layer B.Cu) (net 7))
 (segment (start 123.625 93.92) (end 123.625 95.1875) (width 0.25) (layer B.Cu) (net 7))
 (segment (start 125.16 89.12) (end 125.16 89.205) (width 0.25) (layer F.Cu) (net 7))
 (segment (start 125.16 89.12) (end 125.16 89.205) (width 0.25) (layer F.Cu) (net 7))
 (segment (start 125.16 89.205) (end 125.16 89.295) (width 0.25) (layer F.Cu) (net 7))
 (segment (start 125.16 89.295) (end 124.76 89.695) (width 0.25) (layer F.Cu) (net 7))
 (segment (start 124.76 89.695) (end 124.76 90.0995) (width 0.25) (layer F.Cu) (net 7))
 (segment (start 124.76 90.0995) (end 124.785 90.1245) (width 0.25) (layer F.Cu) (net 7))
 (segment (start 123.62 96.46) (end 124.785 95.295) (width 0.25) (layer B.Cu) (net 7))
 (segment (start 124.785 95.295) (end 124.785 90.1245) (width 0.25) (layer B.Cu) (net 7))
 (via (at 124.785 90.1245) (size 0.6) (layers F.Cu B.Cu) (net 7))
 (segment (start 125.525 90.745) (end 125.525 95.825) (width 0.25) (layer B.Cu) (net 8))
 (segment (start 125.525 95.825) (end 126.16 96.46) (width 0.25) (layer B.Cu) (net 8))
 (segment (start 125.66 89.12) (end 125.66 89.5703) (width 0.25) (layer F.Cu) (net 8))
 (segment (start 125.66 89.5703) (end 125.41 89.8203) (width 0.25) (layer F.Cu) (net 8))
 (segment (start 125.41 89.8203) (end 125.41 90.63) (width 0.25) (layer F.Cu) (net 8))
 (segment (start 125.41 90.63) (end 125.525 90.745) (width 0.25) (layer F.Cu) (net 8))
 (segment (start 123.625 92.015) (end 123.625 90.105) (width 0.25) (layer B.Cu) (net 8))
 (segment (start 123.625 90.105) (end 124.255 89.475) (width 0.25) (layer B.Cu) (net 8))
 (segment (start 124.255 89.475) (end 125.065 89.475) (width 0.25) (layer B.Cu) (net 8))
 (segment (start 125.065 89.475) (end 125.41 89.8203) (width 0.25) (layer B.Cu) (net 8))
 (segment (start 125.41 89.8203) (end 125.41 90.63) (width 0.25) (layer B.Cu) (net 8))
 (segment (start 125.41 90.63) (end 125.525 90.745) (width 0.25) (layer B.Cu) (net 8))
 (via (at 125.525 90.745) (size 0.6) (layers F.Cu B.Cu) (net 8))
 (segment (start 126.66 86.02) (end 126.66 85.3681) (width 0.25) (layer F.Cu) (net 11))
 (segment (start 127.685 82.49) (end 127.685 84.6169) (width 0.25) (layer F.Cu) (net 11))
 (segment (start 127.685 84.6169) (end 127.4112 84.6169) (width 0.25) (layer F.Cu) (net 11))
 (segment (start 127.4112 84.6169) (end 126.66 85.3681) (width 0.25) (layer F.Cu) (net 11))
 (segment (start 125.66 86.02) (end 125.66 85.3681) (width 0.25) (layer F.Cu) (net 12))
 (segment (start 124.635 82.49) (end 124.635 84.6169) (width 0.25) (layer F.Cu) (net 12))
 (segment (start 124.635 84.6169) (end 124.9088 84.6169) (width 0.25) (layer F.Cu) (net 12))
 (segment (start 124.9088 84.6169) (end 125.66 85.3681) (width 0.25) (layer F.Cu) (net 12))
 (segment (start 119.55 94) (end 120.5 94) (width 0.25) (layer F.Cu) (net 9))
 (segment (start 120.5 94) (end 122.26 94) (width 0.25) (layer B.Cu) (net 9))
 (segment (start 122.26 94) (end 122.34 93.92) (width 0.25) (layer B.Cu) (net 9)) (via (at 120.5 94) (size 0.6) (layers F.Cu B.Cu) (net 9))
 (segment (start 119.55 92) (end 120.5 92) (width 0.25) (layer F.Cu) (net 10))
 (segment (start 120.5 92) (end 122.33 92) (width 0.25) (layer B.Cu) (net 10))
 (segment (start 122.33 92) (end 122.345 92.015) (width 0.25) (layer B.Cu) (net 10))
 (via (at 120.5 92) (size 0.6) (layers F.Cu B.Cu) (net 10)))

